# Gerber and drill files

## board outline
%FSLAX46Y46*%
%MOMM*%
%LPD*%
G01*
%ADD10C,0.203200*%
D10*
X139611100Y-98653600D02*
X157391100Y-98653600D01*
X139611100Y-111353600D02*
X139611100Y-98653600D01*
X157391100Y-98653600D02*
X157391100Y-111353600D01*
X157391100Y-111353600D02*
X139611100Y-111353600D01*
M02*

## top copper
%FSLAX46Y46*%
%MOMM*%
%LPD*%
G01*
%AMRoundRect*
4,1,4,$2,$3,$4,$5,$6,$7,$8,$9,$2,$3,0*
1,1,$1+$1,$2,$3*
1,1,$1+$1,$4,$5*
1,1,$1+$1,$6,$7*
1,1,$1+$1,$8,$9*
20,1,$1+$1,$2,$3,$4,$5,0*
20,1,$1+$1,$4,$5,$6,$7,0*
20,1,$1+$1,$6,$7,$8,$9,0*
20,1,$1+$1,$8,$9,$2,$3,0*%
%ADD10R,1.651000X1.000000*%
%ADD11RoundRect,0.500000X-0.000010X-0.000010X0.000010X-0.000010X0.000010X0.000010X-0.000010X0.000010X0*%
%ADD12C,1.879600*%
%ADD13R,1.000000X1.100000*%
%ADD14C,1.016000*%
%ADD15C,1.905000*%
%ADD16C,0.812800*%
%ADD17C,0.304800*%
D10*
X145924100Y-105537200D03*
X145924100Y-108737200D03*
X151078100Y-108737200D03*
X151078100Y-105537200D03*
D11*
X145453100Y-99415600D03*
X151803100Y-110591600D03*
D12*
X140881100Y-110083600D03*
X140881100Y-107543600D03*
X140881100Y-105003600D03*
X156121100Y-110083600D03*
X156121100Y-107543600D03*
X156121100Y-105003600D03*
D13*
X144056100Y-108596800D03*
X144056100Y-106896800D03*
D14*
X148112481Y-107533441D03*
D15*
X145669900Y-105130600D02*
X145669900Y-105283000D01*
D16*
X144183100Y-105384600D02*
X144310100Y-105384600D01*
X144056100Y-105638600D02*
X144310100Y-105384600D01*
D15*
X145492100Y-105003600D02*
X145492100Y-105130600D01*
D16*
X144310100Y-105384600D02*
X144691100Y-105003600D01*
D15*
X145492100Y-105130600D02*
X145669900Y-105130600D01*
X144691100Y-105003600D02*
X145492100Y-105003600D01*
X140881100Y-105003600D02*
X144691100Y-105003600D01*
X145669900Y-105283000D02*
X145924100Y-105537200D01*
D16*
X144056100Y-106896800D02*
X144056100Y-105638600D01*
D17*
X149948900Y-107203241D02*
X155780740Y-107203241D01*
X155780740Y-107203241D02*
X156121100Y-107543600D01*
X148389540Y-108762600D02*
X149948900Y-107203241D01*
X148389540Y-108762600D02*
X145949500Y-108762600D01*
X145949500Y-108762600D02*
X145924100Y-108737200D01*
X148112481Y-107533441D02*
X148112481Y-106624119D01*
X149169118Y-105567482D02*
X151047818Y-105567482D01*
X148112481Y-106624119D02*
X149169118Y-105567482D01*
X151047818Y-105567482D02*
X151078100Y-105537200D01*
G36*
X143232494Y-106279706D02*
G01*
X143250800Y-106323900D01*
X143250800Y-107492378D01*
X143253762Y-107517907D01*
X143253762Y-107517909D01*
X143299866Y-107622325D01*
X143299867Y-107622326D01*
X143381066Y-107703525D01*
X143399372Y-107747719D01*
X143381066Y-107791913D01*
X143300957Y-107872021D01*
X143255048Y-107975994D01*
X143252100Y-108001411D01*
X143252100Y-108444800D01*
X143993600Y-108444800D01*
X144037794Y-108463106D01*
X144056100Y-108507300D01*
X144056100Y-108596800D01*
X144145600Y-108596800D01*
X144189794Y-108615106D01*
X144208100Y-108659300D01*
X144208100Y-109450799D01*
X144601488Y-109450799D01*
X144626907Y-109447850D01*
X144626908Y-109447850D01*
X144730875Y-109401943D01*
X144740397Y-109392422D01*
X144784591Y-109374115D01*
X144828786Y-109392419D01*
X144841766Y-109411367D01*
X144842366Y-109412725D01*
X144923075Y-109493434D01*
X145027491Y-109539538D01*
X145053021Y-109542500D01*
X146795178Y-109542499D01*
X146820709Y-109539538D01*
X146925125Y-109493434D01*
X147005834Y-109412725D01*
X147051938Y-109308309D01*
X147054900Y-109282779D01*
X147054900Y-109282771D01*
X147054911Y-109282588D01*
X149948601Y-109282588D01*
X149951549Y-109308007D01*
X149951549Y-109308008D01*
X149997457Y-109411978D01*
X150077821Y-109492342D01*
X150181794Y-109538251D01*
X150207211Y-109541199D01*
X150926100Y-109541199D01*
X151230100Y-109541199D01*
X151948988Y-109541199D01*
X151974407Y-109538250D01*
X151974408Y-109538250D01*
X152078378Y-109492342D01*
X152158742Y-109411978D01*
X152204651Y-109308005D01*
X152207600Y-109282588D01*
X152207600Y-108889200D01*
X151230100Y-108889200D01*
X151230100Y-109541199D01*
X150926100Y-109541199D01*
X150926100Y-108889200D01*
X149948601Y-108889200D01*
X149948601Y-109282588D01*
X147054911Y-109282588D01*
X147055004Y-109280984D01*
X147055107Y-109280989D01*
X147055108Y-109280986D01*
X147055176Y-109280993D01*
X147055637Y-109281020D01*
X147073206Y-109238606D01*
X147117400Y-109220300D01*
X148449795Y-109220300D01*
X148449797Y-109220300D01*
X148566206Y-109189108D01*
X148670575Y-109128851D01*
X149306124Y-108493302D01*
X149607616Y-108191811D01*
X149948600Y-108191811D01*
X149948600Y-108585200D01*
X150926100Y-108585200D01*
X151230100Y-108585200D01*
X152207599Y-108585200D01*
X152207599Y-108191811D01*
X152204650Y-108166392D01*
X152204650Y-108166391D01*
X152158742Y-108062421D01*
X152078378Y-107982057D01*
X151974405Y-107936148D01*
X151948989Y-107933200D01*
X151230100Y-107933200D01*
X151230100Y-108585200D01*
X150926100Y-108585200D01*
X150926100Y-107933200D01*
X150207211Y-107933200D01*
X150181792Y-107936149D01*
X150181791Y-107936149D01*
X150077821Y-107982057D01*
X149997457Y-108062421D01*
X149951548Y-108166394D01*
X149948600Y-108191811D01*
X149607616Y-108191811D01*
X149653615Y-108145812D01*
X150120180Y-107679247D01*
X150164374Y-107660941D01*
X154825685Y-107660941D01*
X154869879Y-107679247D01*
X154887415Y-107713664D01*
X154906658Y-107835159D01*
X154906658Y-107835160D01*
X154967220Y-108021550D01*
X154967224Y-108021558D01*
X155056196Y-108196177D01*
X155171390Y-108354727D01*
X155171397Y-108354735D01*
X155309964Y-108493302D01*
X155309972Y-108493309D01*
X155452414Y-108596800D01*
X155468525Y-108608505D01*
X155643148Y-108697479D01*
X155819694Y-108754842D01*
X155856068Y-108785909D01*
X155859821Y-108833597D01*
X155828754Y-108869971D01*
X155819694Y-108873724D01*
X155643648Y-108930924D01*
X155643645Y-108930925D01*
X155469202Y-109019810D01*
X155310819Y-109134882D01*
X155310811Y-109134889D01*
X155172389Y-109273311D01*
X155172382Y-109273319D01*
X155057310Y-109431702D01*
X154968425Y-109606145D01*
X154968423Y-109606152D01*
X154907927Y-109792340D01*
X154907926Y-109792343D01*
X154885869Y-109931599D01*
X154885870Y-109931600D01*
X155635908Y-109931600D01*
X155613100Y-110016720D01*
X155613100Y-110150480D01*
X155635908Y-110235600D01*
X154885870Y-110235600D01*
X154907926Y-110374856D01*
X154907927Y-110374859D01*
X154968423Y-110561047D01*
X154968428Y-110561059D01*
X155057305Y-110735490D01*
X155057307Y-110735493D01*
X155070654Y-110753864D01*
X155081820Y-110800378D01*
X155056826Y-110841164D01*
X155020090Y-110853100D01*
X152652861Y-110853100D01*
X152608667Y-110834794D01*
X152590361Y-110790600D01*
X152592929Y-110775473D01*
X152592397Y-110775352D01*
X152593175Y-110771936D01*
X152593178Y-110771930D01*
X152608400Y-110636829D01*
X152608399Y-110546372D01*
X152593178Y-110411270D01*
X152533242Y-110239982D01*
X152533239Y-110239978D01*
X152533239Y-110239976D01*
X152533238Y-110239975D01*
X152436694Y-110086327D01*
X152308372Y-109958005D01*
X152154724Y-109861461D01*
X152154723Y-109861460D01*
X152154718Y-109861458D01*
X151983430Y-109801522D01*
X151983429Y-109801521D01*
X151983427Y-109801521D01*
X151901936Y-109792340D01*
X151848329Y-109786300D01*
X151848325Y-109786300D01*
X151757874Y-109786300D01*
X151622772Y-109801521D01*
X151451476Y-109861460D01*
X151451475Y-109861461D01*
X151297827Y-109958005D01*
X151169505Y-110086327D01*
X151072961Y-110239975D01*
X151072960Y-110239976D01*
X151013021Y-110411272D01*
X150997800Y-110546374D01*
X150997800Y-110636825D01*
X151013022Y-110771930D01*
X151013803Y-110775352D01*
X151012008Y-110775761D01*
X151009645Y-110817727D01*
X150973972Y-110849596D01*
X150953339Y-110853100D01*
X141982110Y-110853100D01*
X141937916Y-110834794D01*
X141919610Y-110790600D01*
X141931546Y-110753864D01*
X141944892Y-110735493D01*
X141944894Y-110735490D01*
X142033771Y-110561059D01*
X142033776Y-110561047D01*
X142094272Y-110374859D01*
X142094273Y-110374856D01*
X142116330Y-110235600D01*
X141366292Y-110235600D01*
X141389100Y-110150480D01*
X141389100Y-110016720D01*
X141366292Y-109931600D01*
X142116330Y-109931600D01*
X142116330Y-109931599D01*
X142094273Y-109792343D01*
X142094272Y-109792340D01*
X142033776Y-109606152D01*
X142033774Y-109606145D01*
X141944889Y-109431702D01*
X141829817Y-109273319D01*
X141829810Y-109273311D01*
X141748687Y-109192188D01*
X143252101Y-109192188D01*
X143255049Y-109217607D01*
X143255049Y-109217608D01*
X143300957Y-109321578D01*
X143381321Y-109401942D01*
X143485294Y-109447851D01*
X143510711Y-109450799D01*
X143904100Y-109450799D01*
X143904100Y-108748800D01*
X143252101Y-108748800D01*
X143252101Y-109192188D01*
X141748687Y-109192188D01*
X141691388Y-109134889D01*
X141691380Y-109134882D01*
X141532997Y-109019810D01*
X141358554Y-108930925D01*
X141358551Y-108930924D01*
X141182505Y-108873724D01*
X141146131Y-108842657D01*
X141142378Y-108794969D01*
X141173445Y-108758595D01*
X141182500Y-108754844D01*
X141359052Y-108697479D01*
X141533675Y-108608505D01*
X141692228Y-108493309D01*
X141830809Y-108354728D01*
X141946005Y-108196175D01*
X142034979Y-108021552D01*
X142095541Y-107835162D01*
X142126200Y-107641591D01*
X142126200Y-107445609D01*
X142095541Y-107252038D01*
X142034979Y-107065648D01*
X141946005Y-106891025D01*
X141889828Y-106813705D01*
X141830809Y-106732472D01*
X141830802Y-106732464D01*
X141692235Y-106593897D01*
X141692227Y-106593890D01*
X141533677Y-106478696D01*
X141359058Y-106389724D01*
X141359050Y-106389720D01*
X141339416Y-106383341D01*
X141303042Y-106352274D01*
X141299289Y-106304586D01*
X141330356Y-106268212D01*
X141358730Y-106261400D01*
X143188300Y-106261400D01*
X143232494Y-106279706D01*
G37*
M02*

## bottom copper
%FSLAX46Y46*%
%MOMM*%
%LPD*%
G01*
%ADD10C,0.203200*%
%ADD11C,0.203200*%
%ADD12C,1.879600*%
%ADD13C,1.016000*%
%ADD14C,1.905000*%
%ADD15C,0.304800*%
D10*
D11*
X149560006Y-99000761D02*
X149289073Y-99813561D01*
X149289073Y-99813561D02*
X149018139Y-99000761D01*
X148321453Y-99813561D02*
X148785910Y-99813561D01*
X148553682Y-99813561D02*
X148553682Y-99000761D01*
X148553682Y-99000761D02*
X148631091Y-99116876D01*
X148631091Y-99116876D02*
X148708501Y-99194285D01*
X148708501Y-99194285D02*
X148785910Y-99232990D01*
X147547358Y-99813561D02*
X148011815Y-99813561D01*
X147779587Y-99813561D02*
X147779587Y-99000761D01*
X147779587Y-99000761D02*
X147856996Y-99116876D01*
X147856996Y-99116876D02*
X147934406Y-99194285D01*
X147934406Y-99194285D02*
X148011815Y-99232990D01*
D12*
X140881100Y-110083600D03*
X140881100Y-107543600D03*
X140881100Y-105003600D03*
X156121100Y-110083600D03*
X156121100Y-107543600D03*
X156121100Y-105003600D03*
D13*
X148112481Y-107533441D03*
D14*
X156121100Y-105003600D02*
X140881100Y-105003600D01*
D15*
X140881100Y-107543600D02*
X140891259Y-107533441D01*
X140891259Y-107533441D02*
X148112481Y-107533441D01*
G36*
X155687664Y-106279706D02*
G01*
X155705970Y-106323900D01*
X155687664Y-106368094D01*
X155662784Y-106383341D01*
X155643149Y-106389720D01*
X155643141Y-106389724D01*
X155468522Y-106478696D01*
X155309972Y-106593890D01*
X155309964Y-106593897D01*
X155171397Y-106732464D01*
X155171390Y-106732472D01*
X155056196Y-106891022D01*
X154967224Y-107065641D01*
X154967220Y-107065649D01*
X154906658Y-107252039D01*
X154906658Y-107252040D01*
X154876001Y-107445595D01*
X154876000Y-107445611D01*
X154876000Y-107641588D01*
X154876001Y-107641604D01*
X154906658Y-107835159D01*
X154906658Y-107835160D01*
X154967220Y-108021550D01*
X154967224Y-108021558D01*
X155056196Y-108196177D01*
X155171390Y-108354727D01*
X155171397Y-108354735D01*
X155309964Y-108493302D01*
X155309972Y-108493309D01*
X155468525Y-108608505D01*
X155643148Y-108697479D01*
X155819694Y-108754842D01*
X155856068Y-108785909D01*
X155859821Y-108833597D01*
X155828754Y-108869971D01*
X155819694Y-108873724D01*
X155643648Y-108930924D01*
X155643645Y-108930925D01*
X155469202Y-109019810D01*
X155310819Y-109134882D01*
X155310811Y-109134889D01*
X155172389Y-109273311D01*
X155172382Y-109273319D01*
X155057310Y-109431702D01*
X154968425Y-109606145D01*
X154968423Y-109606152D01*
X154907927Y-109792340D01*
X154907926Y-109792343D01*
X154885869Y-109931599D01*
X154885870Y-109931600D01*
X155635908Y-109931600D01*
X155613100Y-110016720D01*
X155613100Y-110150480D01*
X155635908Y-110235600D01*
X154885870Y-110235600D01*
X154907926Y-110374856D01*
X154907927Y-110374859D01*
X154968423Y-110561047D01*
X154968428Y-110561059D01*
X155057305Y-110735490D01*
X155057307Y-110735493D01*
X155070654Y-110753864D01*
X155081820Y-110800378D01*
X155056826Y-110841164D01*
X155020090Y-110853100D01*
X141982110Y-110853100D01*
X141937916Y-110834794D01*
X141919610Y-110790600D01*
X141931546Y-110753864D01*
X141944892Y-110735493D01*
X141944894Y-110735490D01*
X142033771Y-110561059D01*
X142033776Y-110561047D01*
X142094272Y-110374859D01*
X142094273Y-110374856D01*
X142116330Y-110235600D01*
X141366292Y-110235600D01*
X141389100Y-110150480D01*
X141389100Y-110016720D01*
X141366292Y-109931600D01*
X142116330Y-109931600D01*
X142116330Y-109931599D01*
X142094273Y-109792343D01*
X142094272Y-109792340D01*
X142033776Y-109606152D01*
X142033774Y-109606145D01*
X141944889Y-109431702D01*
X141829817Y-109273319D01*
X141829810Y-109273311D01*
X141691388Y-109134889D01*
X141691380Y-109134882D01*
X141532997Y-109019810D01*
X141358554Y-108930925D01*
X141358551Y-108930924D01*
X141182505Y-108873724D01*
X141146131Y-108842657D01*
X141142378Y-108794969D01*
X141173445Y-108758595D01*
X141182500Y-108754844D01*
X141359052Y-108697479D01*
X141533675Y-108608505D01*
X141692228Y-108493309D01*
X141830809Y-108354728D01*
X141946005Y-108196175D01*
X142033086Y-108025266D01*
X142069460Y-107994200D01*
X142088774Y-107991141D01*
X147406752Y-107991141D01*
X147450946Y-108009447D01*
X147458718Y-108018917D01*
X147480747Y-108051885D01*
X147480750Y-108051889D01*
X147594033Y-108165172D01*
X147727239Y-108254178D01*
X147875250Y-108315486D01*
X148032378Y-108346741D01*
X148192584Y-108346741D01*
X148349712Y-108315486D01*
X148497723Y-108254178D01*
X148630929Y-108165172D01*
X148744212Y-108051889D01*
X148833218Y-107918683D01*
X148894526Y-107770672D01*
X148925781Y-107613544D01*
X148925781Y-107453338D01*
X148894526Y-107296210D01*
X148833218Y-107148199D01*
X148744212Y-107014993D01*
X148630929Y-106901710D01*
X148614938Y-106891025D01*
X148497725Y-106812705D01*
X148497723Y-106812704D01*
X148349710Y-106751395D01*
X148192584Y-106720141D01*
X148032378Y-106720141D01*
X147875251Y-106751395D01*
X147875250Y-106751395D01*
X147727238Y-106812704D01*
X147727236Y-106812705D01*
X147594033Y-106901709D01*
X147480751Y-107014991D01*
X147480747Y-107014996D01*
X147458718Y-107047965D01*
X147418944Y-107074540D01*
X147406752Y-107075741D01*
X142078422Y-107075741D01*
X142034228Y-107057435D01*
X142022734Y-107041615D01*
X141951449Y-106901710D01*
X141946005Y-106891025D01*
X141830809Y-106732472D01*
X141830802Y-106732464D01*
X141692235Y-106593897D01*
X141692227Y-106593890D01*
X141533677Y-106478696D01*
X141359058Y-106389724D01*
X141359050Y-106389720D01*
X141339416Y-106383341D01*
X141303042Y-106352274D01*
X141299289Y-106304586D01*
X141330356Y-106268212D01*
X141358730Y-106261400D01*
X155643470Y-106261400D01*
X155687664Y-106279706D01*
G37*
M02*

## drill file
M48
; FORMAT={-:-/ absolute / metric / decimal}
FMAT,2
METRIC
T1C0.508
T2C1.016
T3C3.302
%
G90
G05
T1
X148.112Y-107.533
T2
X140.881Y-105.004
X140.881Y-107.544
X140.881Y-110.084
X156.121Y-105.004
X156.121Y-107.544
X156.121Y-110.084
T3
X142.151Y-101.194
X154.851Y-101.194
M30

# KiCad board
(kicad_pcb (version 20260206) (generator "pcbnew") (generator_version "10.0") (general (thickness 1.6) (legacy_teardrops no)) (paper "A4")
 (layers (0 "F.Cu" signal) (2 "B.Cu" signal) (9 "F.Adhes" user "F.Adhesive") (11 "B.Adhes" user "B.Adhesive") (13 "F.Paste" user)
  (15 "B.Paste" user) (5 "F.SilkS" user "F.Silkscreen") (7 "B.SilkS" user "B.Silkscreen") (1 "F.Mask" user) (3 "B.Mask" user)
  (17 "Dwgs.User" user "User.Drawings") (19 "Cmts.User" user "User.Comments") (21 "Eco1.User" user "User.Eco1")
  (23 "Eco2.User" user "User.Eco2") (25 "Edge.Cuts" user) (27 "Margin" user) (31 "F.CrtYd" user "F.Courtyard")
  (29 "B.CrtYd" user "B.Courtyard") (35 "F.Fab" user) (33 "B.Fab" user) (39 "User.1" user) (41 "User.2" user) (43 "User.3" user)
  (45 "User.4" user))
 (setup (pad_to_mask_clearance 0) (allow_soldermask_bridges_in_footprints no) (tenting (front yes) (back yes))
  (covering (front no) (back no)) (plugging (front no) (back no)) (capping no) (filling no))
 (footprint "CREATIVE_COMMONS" (layer "F.Cu") (at 118.159513 124.0536)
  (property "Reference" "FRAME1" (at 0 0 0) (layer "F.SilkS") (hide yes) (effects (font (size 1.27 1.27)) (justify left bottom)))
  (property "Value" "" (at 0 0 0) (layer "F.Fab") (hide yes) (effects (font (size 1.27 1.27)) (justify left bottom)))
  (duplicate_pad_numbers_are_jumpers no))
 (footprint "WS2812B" (layer "F.Cu") (at 148.5011 107.1372)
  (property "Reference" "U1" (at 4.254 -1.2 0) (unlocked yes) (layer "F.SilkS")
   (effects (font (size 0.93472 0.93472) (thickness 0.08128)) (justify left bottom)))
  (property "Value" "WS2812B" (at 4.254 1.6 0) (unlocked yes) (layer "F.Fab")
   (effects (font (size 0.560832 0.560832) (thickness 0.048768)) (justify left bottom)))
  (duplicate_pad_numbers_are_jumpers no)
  (pad "1" smd rect (at -2.577 -1.6) (size 1.651 1) (layers "F.Cu" "F.Mask" "F.Paste") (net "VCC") (solder_mask_margin 0.1016)
   (solder_paste_margin 0) (thermal_bridge_angle 0))
  (pad "2" smd rect (at -2.577 1.6) (size 1.651 1) (layers "F.Cu" "F.Mask" "F.Paste") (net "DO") (solder_mask_margin 0.1016)
   (solder_paste_margin 0) (thermal_bridge_angle 0))
  (pad "3" smd rect (at 2.577 1.6) (size 1.651 1) (layers "F.Cu" "F.Mask" "F.Paste") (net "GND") (solder_mask_margin 0.1016)
   (solder_paste_margin 0) (thermal_bridge_angle 0))
  (pad "4" smd rect (at 2.577 -1.6) (size 1.651 1) (layers "F.Cu" "F.Mask" "F.Paste") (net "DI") (solder_mask_margin 0.1016)
   (solder_paste_margin 0) (thermal_bridge_angle 0)))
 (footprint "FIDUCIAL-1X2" (layer "F.Cu") (at 145.4531 99.4156)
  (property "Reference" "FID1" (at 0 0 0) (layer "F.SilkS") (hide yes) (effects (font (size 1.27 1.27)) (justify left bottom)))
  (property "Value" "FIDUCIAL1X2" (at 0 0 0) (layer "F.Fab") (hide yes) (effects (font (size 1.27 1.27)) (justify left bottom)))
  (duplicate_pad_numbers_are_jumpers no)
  (pad "1" smd roundrect (at 0 0) (size 1 1) (layers "F.Cu" "F.Mask") (roundrect_rratio 0.5) (solder_mask_margin 0.1016)
   (solder_paste_margin 0) (thermal_bridge_angle 0)))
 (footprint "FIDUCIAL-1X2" (layer "F.Cu") (at 151.8031 110.5916)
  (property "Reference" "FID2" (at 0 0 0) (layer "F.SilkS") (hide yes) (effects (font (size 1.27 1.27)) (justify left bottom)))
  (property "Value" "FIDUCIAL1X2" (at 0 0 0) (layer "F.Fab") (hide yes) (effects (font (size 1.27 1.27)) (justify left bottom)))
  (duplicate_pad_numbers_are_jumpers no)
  (pad "1" smd roundrect (at 0 0) (size 1 1) (layers "F.Cu" "F.Mask") (roundrect_rratio 0.5) (solder_mask_margin 0.1016)
   (solder_paste_margin 0) (thermal_bridge_angle 0)))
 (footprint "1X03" (layer "F.Cu") (at 140.8811 110.0836 90)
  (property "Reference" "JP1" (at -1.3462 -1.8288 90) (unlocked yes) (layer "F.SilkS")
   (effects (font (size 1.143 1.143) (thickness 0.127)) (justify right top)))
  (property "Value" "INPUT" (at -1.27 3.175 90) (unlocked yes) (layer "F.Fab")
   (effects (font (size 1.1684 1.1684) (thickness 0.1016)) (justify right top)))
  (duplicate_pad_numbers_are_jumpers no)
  (pad "1" thru_hole circle (at 0 0 180) (size 1.8796 1.8796) (drill 1.016) (layers "*.Cu" "*.Mask") (remove_unused_layers no) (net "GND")
   (solder_mask_margin 0.1016) (thermal_bridge_angle 0))
  (pad "2" thru_hole circle (at 2.54 0 180) (size 1.8796 1.8796) (drill 1.016) (layers "*.Cu" "*.Mask") (remove_unused_layers no) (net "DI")
   (solder_mask_margin 0.1016) (thermal_bridge_angle 0))
  (pad "3" thru_hole circle (at 5.08 0 180) (size 1.8796 1.8796) (drill 1.016) (layers "*.Cu" "*.Mask") (remove_unused_layers no)
   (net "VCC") (solder_mask_margin 0.1016) (thermal_bridge_angle 0)))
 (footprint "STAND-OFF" (layer "F.Cu") (at 154.8511 101.1936)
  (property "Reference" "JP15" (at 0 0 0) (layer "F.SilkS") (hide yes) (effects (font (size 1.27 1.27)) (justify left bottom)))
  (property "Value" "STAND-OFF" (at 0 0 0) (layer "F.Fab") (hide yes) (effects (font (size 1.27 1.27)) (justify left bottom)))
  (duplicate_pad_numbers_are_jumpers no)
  (pad "" np_thru_hole circle (at 0 0) (size 3.302 3.302) (drill 3.302) (layers "*.Cu" "*.Mask")))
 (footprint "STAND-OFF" (layer "F.Cu") (at 142.1511 101.1936)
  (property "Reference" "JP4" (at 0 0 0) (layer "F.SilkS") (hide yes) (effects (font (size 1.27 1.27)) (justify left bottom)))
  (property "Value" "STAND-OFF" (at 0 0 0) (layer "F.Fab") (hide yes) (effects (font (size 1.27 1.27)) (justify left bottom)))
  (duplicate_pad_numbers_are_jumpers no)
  (pad "" np_thru_hole circle (at 0 0) (size 3.302 3.302) (drill 3.302) (layers "*.Cu" "*.Mask")))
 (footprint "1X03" (layer "F.Cu") (at 156.1211 110.0836 90)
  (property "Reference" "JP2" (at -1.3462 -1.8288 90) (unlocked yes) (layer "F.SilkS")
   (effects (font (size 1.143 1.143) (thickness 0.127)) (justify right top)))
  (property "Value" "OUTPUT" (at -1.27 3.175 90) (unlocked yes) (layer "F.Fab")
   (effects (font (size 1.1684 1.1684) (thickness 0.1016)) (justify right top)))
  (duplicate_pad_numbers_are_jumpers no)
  (pad "1" thru_hole circle (at 0 0 180) (size 1.8796 1.8796) (drill 1.016) (layers "*.Cu" "*.Mask") (remove_unused_layers no) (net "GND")
   (solder_mask_margin 0.1016) (thermal_bridge_angle 0))
  (pad "2" thru_hole circle (at 2.54 0 180) (size 1.8796 1.8796) (drill 1.016) (layers "*.Cu" "*.Mask") (remove_unused_layers no) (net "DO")
   (solder_mask_margin 0.1016) (thermal_bridge_angle 0))
  (pad "3" thru_hole circle (at 5.08 0 180) (size 1.8796 1.8796) (drill 1.016) (layers "*.Cu" "*.Mask") (remove_unused_layers no)
   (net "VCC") (solder_mask_margin 0.1016) (thermal_bridge_angle 0)))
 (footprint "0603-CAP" (layer "F.Cu") (at 144.0561 107.7468 90)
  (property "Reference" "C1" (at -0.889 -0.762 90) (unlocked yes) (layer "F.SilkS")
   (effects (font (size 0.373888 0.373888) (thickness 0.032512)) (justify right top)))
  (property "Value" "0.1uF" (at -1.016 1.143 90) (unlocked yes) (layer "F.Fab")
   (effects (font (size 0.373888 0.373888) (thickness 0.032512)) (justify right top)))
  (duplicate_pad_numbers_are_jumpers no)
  (pad "1" smd rect (at -0.85 0 90) (size 1.1 1) (layers "F.Cu" "F.Mask" "F.Paste") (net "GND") (solder_mask_margin 0.1016)
   (solder_paste_margin 0) (thermal_bridge_angle 0))
  (pad "2" smd rect (at 0.85 0 90) (size 1.1 1) (layers "F.Cu" "F.Mask" "F.Paste") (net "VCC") (solder_mask_margin 0.1016)
   (solder_paste_margin 0) (thermal_bridge_angle 0)))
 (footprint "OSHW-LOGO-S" (layer "B.Cu") (at 148.587459 102.217222 180)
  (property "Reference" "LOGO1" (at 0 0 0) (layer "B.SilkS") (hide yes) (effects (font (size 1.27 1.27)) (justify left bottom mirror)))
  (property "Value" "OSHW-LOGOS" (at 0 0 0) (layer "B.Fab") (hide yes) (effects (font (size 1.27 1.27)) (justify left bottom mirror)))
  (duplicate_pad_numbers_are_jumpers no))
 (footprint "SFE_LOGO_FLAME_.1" (layer "B.Cu") (at 149.768559 106.913679 180)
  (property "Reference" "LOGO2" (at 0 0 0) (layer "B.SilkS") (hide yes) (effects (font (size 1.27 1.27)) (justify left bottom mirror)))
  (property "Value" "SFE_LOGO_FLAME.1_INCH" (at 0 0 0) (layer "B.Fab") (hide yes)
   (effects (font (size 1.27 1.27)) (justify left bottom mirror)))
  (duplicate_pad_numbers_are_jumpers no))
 (gr_line (start 139.6111 98.6536) (end 157.3911 98.6536) (stroke (width 0.2032) (type solid)) (layer "Edge.Cuts"))
 (gr_line (start 139.6111 111.3536) (end 139.6111 98.6536) (stroke (width 0.2032) (type solid)) (layer "Edge.Cuts"))
 (gr_line (start 157.3911 98.6536) (end 157.3911 111.3536) (stroke (width 0.2032) (type solid)) (layer "Edge.Cuts"))
 (gr_line (start 157.3911 111.3536) (end 139.6111 111.3536) (stroke (width 0.2032) (type solid)) (layer "Edge.Cuts"))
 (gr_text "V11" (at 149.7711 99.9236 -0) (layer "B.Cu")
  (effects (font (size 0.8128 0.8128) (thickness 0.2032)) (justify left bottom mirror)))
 (segment (start 145.6699 105.1306) (end 145.6699 105.283) (width 1.905) (layer "F.Cu") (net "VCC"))
 (segment (start 144.1831 105.3846) (end 144.3101 105.3846) (width 0.8128) (layer "F.Cu") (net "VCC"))
 (segment (start 144.0561 105.6386) (end 144.3101 105.3846) (width 0.8128) (layer "F.Cu") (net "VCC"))
 (segment (start 145.4921 105.0036) (end 145.4921 105.1306) (width 1.905) (layer "F.Cu") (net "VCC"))
 (segment (start 144.3101 105.3846) (end 144.6911 105.0036) (width 0.8128) (layer "F.Cu") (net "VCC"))
 (segment (start 145.4921 105.1306) (end 145.6699 105.1306) (width 1.905) (layer "F.Cu") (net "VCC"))
 (segment (start 144.6911 105.0036) (end 145.4921 105.0036) (width 1.905) (layer "F.Cu") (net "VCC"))
 (segment (start 140.8811 105.0036) (end 144.6911 105.0036) (width 1.905) (layer "F.Cu") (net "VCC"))
 (segment (start 145.6699 105.283) (end 145.9241 105.5372) (width 1.905) (layer "F.Cu") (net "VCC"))
 (segment (start 144.0561 106.8968) (end 144.0561 105.6386) (width 0.8128) (layer "F.Cu") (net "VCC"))
 (segment (start 156.1211 105.0036) (end 140.8811 105.0036) (width 1.905) (layer "B.Cu") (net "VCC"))
 (segment (start 149.9489 107.203241) (end 155.78074 107.203241) (width 0.3048) (layer "F.Cu") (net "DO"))
 (segment (start 155.78074 107.203241) (end 156.1211 107.5436) (width 0.3048) (layer "F.Cu") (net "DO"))
 (segment (start 148.38954 108.7626) (end 149.9489 107.203241) (width 0.3048) (layer "F.Cu") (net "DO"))
 (segment (start 148.38954 108.7626) (end 145.9495 108.7626) (width 0.3048) (layer "F.Cu") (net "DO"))
 (segment (start 145.9495 108.7626) (end 145.9241 108.7372) (width 0.3048) (layer "F.Cu") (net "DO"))
 (segment (start 148.112481 107.533441) (end 148.112481 106.624119) (width 0.3048) (layer "F.Cu") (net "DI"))
 (segment (start 149.169118 105.567482) (end 151.047818 105.567482) (width 0.3048) (layer "F.Cu") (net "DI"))
 (segment (start 148.112481 106.624119) (end 149.169118 105.567482) (width 0.3048) (layer "F.Cu") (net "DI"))
 (segment (start 151.047818 105.567482) (end 151.0781 105.5372) (width 0.3048) (layer "F.Cu") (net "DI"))
 (via (at 148.112481 107.533441) (size 1.016) (drill 0.508) (layers "F.Cu" "B.Cu") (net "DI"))
 (segment (start 140.8811 107.5436) (end 140.891259 107.533441) (width 0.3048) (layer "B.Cu") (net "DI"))
 (segment (start 140.891259 107.533441) (end 148.112481 107.533441) (width 0.3048) (layer "B.Cu") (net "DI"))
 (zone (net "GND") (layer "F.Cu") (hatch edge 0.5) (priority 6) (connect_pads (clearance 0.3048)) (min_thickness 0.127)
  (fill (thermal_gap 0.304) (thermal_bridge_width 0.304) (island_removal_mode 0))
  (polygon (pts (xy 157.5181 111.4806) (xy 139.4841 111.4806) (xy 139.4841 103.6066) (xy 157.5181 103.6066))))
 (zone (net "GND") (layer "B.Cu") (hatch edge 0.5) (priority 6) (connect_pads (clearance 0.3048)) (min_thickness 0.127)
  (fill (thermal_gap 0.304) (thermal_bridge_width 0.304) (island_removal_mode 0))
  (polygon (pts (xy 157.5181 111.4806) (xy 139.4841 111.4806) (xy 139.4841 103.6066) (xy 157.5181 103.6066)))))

